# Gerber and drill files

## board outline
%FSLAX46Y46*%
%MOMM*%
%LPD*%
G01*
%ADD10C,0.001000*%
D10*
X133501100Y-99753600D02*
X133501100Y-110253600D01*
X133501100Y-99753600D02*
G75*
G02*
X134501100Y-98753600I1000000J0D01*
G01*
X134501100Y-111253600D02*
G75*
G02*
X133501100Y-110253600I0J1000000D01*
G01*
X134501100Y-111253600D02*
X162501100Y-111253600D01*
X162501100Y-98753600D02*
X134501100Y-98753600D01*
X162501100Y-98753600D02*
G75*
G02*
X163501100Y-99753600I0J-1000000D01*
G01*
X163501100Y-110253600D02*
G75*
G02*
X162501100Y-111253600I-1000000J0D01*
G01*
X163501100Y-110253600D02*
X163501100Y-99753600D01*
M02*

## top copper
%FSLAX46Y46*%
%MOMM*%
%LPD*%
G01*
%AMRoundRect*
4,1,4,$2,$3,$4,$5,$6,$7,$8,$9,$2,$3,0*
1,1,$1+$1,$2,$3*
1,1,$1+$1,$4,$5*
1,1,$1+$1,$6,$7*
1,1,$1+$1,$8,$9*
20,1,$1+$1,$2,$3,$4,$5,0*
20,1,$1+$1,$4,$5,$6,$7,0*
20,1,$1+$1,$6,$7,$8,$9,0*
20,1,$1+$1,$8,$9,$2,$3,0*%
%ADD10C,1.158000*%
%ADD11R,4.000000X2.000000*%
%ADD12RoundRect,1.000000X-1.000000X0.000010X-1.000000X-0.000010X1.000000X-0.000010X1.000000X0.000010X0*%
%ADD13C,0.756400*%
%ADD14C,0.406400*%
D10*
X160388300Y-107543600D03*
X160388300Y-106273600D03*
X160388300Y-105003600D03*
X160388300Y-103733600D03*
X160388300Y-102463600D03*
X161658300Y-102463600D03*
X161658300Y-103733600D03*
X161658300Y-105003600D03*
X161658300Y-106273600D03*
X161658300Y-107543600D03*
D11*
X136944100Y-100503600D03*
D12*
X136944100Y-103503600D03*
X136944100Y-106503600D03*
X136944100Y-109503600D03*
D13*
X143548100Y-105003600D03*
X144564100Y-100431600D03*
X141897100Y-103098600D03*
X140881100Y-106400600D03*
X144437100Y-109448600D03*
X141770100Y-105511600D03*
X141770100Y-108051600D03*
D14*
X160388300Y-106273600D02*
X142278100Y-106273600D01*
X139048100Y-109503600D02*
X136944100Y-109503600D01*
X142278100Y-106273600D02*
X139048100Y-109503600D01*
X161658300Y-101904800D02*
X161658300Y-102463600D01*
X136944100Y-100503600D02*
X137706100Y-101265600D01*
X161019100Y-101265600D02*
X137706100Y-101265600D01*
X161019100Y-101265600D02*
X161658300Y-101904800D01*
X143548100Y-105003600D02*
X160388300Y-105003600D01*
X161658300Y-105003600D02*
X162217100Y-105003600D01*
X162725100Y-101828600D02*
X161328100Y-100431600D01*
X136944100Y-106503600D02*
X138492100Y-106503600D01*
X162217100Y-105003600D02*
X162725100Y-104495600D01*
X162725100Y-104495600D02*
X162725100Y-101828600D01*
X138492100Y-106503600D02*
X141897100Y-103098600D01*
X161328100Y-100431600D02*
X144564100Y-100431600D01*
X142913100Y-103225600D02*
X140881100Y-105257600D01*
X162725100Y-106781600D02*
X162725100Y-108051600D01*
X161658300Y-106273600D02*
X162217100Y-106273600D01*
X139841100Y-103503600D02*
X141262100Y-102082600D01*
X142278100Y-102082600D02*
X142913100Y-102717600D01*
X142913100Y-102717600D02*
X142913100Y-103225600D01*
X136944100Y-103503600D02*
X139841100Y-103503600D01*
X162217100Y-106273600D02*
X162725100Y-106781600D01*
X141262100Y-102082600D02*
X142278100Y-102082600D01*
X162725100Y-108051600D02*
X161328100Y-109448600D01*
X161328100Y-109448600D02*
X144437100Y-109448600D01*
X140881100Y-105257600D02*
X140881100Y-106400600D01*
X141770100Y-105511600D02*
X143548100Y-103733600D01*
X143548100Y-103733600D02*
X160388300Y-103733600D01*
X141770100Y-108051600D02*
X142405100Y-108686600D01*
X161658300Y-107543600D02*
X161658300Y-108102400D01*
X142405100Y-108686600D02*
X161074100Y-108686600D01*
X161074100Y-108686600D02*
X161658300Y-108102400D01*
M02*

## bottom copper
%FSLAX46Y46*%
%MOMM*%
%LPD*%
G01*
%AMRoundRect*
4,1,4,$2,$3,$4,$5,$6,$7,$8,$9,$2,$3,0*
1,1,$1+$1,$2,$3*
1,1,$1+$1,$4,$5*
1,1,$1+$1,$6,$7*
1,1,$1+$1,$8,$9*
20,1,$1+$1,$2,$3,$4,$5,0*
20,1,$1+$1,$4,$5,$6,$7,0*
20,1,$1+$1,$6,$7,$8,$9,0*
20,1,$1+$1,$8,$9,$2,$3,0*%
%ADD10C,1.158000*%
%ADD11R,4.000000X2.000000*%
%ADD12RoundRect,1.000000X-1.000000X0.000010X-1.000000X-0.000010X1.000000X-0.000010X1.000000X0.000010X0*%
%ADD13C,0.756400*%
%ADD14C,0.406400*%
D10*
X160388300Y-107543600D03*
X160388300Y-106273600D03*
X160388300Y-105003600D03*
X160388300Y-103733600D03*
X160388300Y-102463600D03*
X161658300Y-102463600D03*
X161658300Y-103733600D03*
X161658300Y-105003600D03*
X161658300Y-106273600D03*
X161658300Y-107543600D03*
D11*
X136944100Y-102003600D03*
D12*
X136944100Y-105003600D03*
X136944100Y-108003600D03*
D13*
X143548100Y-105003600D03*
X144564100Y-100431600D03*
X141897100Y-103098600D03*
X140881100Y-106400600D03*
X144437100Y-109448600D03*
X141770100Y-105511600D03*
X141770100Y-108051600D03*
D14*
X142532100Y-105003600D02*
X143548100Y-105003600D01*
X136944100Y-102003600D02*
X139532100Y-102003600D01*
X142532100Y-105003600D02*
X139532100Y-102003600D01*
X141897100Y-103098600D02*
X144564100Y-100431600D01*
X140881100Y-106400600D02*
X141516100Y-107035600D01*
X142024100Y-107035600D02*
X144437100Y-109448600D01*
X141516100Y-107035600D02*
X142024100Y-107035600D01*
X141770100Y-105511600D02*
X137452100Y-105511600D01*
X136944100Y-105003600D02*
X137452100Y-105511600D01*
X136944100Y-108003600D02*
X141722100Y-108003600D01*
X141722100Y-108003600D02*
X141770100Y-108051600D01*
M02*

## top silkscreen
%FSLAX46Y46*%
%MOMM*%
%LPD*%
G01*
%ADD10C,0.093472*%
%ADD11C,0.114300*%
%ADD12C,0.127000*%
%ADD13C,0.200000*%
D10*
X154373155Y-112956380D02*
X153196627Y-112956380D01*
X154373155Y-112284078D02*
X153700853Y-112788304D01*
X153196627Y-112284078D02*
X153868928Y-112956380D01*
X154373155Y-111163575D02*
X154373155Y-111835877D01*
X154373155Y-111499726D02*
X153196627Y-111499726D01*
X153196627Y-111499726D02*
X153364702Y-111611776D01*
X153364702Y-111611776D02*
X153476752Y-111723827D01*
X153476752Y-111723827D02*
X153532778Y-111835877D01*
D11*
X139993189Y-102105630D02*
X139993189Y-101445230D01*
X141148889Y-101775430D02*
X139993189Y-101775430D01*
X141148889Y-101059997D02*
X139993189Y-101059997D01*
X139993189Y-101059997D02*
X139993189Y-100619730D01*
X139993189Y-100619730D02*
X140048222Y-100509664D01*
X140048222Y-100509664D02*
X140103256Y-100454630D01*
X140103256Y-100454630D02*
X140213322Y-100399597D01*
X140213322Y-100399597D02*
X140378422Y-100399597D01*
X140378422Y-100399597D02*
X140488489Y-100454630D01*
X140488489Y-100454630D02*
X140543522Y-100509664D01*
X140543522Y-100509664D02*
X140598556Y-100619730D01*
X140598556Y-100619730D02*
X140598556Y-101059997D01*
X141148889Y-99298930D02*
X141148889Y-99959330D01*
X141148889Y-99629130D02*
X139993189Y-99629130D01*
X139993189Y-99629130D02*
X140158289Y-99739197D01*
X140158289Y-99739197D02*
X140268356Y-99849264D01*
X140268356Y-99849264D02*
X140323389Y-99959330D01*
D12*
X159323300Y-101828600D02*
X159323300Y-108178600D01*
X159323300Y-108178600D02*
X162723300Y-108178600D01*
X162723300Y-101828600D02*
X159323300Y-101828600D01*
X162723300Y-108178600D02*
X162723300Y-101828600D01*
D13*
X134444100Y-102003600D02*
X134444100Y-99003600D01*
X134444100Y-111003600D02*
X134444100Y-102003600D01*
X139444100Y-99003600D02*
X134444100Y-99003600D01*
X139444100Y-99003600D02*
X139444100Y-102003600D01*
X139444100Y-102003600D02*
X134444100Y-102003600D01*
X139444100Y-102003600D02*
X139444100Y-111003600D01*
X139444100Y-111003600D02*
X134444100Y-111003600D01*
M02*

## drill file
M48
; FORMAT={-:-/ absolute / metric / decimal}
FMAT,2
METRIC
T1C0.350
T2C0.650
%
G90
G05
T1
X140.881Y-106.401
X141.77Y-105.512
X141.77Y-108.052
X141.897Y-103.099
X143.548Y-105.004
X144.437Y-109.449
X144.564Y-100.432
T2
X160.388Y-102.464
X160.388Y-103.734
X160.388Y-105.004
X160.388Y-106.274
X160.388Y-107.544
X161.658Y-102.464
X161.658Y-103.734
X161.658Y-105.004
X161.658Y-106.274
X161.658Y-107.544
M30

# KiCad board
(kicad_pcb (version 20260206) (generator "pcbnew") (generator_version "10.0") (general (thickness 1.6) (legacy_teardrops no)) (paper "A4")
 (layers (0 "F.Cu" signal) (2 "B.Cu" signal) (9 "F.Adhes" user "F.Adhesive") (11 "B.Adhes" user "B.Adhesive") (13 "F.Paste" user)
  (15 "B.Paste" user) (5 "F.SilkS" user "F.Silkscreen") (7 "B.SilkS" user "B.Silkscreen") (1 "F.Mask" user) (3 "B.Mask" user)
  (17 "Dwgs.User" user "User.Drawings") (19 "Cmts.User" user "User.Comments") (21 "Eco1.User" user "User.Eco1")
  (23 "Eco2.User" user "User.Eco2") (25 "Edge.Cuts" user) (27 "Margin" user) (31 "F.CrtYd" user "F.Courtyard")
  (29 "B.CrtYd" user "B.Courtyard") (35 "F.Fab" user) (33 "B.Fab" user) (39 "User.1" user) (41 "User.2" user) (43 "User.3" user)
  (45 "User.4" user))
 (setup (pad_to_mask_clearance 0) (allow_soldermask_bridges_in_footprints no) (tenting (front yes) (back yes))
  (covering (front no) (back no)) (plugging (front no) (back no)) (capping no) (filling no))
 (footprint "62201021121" (layer "F.Cu") (at 161.0233 105.0036 90)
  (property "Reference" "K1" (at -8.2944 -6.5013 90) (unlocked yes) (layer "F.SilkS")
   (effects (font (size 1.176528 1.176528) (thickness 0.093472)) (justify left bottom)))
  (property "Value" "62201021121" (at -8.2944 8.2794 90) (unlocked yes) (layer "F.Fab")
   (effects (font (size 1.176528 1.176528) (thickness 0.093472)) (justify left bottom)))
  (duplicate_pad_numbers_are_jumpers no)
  (fp_line (start 3.175 -1.7) (end -3.175 -1.7) (stroke (width 0.127) (type solid)) (layer "F.SilkS"))
  (fp_line (start -3.175 -1.7) (end -3.175 1.7) (stroke (width 0.127) (type solid)) (layer "F.SilkS"))
  (fp_line (start 3.175 1.7) (end 3.175 -1.7) (stroke (width 0.127) (type solid)) (layer "F.SilkS"))
  (fp_line (start -3.175 1.7) (end 3.175 1.7) (stroke (width 0.127) (type solid)) (layer "F.SilkS"))
  (pad "1" thru_hole circle (at -2.54 -0.635 90) (size 1.158 1.158) (drill 0.65) (layers "*.Cu" "*.Mask") (remove_unused_layers no)
   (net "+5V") (solder_mask_margin 0.1016) (thermal_bridge_angle 0))
  (pad "2" thru_hole circle (at -1.27 -0.635 90) (size 1.158 1.158) (drill 0.65) (layers "*.Cu" "*.Mask") (remove_unused_layers no)
   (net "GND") (solder_mask_margin 0.1016) (thermal_bridge_angle 0))
  (pad "3" thru_hole circle (at 0 -0.635 90) (size 1.158 1.158) (drill 0.65) (layers "*.Cu" "*.Mask") (remove_unused_layers no)
   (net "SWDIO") (solder_mask_margin 0.1016) (thermal_bridge_angle 0))
  (pad "4" thru_hole circle (at 1.27 -0.635 90) (size 1.158 1.158) (drill 0.65) (layers "*.Cu" "*.Mask") (remove_unused_layers no)
   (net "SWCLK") (solder_mask_margin 0.1016) (thermal_bridge_angle 0))
  (pad "5" thru_hole circle (at 2.54 -0.635 90) (size 1.158 1.158) (drill 0.65) (layers "*.Cu" "*.Mask") (remove_unused_layers no)
   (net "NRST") (solder_mask_margin 0.1016) (thermal_bridge_angle 0))
  (pad "6" thru_hole circle (at 2.54 0.635 90) (size 1.158 1.158) (drill 0.65) (layers "*.Cu" "*.Mask") (remove_unused_layers no)
   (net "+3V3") (solder_mask_margin 0.1016) (thermal_bridge_angle 0))
  (pad "7" thru_hole circle (at 1.27 0.635 90) (size 1.158 1.158) (drill 0.65) (layers "*.Cu" "*.Mask") (remove_unused_layers no)
   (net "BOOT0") (solder_mask_margin 0.1016) (thermal_bridge_angle 0))
  (pad "8" thru_hole circle (at 0 0.635 90) (size 1.158 1.158) (drill 0.65) (layers "*.Cu" "*.Mask") (remove_unused_layers no)
   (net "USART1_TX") (solder_mask_margin 0.1016) (thermal_bridge_angle 0))
  (pad "9" thru_hole circle (at -1.27 0.635 90) (size 1.158 1.158) (drill 0.65) (layers "*.Cu" "*.Mask") (remove_unused_layers no)
   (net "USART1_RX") (solder_mask_margin 0.1016) (thermal_bridge_angle 0))
  (pad "10" thru_hole circle (at -2.54 0.635 90) (size 1.158 1.158) (drill 0.65) (layers "*.Cu" "*.Mask") (remove_unused_layers no)
   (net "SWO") (solder_mask_margin 0.1016) (thermal_bridge_angle 0)))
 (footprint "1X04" (layer "F.Cu") (at 136.9441 105.0036 -90)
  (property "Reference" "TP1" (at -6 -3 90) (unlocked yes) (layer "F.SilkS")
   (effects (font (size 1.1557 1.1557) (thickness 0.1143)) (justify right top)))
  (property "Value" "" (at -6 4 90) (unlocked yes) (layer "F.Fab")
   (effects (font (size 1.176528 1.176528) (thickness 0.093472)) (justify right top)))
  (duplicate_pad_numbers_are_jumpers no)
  (fp_line (start -3 2.5) (end -6 2.5) (stroke (width 0.2) (type solid)) (layer "F.SilkS"))
  (fp_line (start 6 2.5) (end -3 2.5) (stroke (width 0.2) (type solid)) (layer "F.SilkS"))
  (fp_line (start -6 -2.5) (end -6 2.5) (stroke (width 0.2) (type solid)) (layer "F.SilkS"))
  (fp_line (start -6 -2.5) (end -3 -2.5) (stroke (width 0.2) (type solid)) (layer "F.SilkS"))
  (fp_line (start -3 -2.5) (end -3 2.5) (stroke (width 0.2) (type solid)) (layer "F.SilkS"))
  (fp_line (start -3 -2.5) (end 6 -2.5) (stroke (width 0.2) (type solid)) (layer "F.SilkS"))
  (fp_line (start 6 -2.5) (end 6 2.5) (stroke (width 0.2) (type solid)) (layer "F.SilkS"))
  (pad "1" smd rect (at -4.5 0 270) (size 2 4) (layers "F.Cu" "F.Mask" "F.Paste") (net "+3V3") (solder_mask_margin 0.1016)
   (solder_paste_margin 0) (thermal_bridge_angle 0))
  (pad "2" smd roundrect (at -1.5 0 270) (size 2 4) (layers "F.Cu" "F.Mask" "F.Paste") (roundrect_rratio 0.5) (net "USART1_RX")
   (solder_mask_margin 0.1016) (solder_paste_margin 0) (thermal_bridge_angle 0))
  (pad "3" smd roundrect (at 1.5 0 270) (size 2 4) (layers "F.Cu" "F.Mask" "F.Paste") (roundrect_rratio 0.5) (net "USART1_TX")
   (solder_mask_margin 0.1016) (solder_paste_margin 0) (thermal_bridge_angle 0))
  (pad "4" smd roundrect (at 4.5 0 270) (size 2 4) (layers "F.Cu" "F.Mask" "F.Paste") (roundrect_rratio 0.5) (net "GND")
   (solder_mask_margin 0.1016) (solder_paste_margin 0) (thermal_bridge_angle 0)))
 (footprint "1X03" (layer "B.Cu") (at 136.9441 105.0036 -90)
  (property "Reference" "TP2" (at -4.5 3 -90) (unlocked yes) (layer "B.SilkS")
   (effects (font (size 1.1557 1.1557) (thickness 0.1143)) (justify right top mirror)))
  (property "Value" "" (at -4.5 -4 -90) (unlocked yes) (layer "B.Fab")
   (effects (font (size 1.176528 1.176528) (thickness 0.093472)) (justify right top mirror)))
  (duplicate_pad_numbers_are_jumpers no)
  (pad "1" smd rect (at -3 0 270) (size 2 4) (layers "B.Cu" "B.Mask" "B.Paste") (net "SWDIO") (solder_mask_margin 0.1016)
   (solder_paste_margin 0) (thermal_bridge_angle 0))
  (pad "2" smd roundrect (at 0 0 270) (size 2 4) (layers "B.Cu" "B.Mask" "B.Paste") (roundrect_rratio 0.5) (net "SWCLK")
   (solder_mask_margin 0.1016) (solder_paste_margin 0) (thermal_bridge_angle 0))
  (pad "3" smd roundrect (at 3 0 270) (size 2 4) (layers "B.Cu" "B.Mask" "B.Paste") (roundrect_rratio 0.5) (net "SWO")
   (solder_mask_margin 0.1016) (solder_paste_margin 0) (thermal_bridge_angle 0)))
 (gr_line (start 133.5011 99.7536) (end 133.5011 110.2536) (stroke (width 0.001) (type solid)) (layer "Edge.Cuts"))
 (gr_arc (start 133.5011 99.7536) (mid 133.793993 99.046493) (end 134.5011 98.7536) (stroke (width 0.001) (type solid)) (layer "Edge.Cuts"))
 (gr_arc (start 134.5011 111.2536) (mid 133.793993 110.960707) (end 133.5011 110.2536) (stroke (width 0.001) (type solid))
  (layer "Edge.Cuts"))
 (gr_line (start 134.5011 111.2536) (end 162.5011 111.2536) (stroke (width 0.001) (type solid)) (layer "Edge.Cuts"))
 (gr_line (start 162.5011 98.7536) (end 134.5011 98.7536) (stroke (width 0.001) (type solid)) (layer "Edge.Cuts"))
 (gr_arc (start 162.5011 98.7536) (mid 163.208207 99.046493) (end 163.5011 99.7536) (stroke (width 0.001) (type solid)) (layer "Edge.Cuts"))
 (gr_arc (start 163.5011 110.2536) (mid 163.208207 110.960707) (end 162.5011 111.2536) (stroke (width 0.001) (type solid))
  (layer "Edge.Cuts"))
 (gr_line (start 163.5011 110.2536) (end 163.5011 99.7536) (stroke (width 0.001) (type solid)) (layer "Edge.Cuts"))
 (segment (start 160.3883 106.2736) (end 142.2781 106.2736) (width 0.4064) (layer "F.Cu") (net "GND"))
 (segment (start 139.0481 109.5036) (end 136.9441 109.5036) (width 0.4064) (layer "F.Cu") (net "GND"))
 (segment (start 142.2781 106.2736) (end 139.0481 109.5036) (width 0.4064) (layer "F.Cu") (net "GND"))
 (segment (start 161.6583 101.9048) (end 161.6583 102.4636) (width 0.4064) (layer "F.Cu") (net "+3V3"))
 (segment (start 136.9441 100.5036) (end 137.7061 101.2656) (width 0.4064) (layer "F.Cu") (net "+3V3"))
 (segment (start 161.0191 101.2656) (end 137.7061 101.2656) (width 0.4064) (layer "F.Cu") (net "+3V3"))
 (segment (start 161.0191 101.2656) (end 161.6583 101.9048) (width 0.4064) (layer "F.Cu") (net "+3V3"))
 (segment (start 143.5481 105.0036) (end 160.3883 105.0036) (width 0.4064) (layer "F.Cu") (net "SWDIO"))
 (via (at 143.5481 105.0036) (size 0.7564) (drill 0.35) (layers "F.Cu" "B.Cu") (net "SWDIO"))
 (segment (start 142.5321 105.0036) (end 143.5481 105.0036) (width 0.4064) (layer "B.Cu") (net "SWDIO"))
 (segment (start 136.9441 102.0036) (end 139.5321 102.0036) (width 0.4064) (layer "B.Cu") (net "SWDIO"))
 (segment (start 142.5321 105.0036) (end 139.5321 102.0036) (width 0.4064) (layer "B.Cu") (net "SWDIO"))
 (segment (start 161.6583 105.0036) (end 162.2171 105.0036) (width 0.4064) (layer "F.Cu") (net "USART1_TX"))
 (segment (start 162.7251 101.8286) (end 161.3281 100.4316) (width 0.4064) (layer "F.Cu") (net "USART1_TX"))
 (segment (start 136.9441 106.5036) (end 138.4921 106.5036) (width 0.4064) (layer "F.Cu") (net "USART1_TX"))
 (segment (start 162.2171 105.0036) (end 162.7251 104.4956) (width 0.4064) (layer "F.Cu") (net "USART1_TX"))
 (segment (start 162.7251 104.4956) (end 162.7251 101.8286) (width 0.4064) (layer "F.Cu") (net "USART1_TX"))
 (segment (start 138.4921 106.5036) (end 141.8971 103.0986) (width 0.4064) (layer "F.Cu") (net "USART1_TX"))
 (segment (start 161.3281 100.4316) (end 144.5641 100.4316) (width 0.4064) (layer "F.Cu") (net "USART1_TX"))
 (via (at 144.5641 100.4316) (size 0.7564) (drill 0.35) (layers "F.Cu" "B.Cu") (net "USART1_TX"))
 (via (at 141.8971 103.0986) (size 0.7564) (drill 0.35) (layers "F.Cu" "B.Cu") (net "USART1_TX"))
 (segment (start 141.8971 103.0986) (end 144.5641 100.4316) (width 0.4064) (layer "B.Cu") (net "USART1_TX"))
 (segment (start 142.9131 103.2256) (end 140.8811 105.2576) (width 0.4064) (layer "F.Cu") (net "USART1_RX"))
 (segment (start 162.7251 106.7816) (end 162.7251 108.0516) (width 0.4064) (layer "F.Cu") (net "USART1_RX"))
 (segment (start 161.6583 106.2736) (end 162.2171 106.2736) (width 0.4064) (layer "F.Cu") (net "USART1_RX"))
 (segment (start 139.8411 103.5036) (end 141.2621 102.0826) (width 0.4064) (layer "F.Cu") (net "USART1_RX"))
 (segment (start 142.2781 102.0826) (end 142.9131 102.7176) (width 0.4064) (layer "F.Cu") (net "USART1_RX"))
 (segment (start 142.9131 102.7176) (end 142.9131 103.2256) (width 0.4064) (layer "F.Cu") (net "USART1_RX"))
 (segment (start 136.9441 103.5036) (end 139.8411 103.5036) (width 0.4064) (layer "F.Cu") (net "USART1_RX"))
 (segment (start 162.2171 106.2736) (end 162.7251 106.7816) (width 0.4064) (layer "F.Cu") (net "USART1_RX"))
 (segment (start 141.2621 102.0826) (end 142.2781 102.0826) (width 0.4064) (layer "F.Cu") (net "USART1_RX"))
 (segment (start 162.7251 108.0516) (end 161.3281 109.4486) (width 0.4064) (layer "F.Cu") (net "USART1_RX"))
 (segment (start 161.3281 109.4486) (end 144.4371 109.4486) (width 0.4064) (layer "F.Cu") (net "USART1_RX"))
 (segment (start 140.8811 105.2576) (end 140.8811 106.4006) (width 0.4064) (layer "F.Cu") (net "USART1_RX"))
 (via (at 140.8811 106.4006) (size 0.7564) (drill 0.35) (layers "F.Cu" "B.Cu") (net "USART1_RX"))
 (via (at 144.4371 109.4486) (size 0.7564) (drill 0.35) (layers "F.Cu" "B.Cu") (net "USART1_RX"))
 (segment (start 140.8811 106.4006) (end 141.5161 107.0356) (width 0.4064) (layer "B.Cu") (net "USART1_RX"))
 (segment (start 142.0241 107.0356) (end 144.4371 109.4486) (width 0.4064) (layer "B.Cu") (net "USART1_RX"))
 (segment (start 141.5161 107.0356) (end 142.0241 107.0356) (width 0.4064) (layer "B.Cu") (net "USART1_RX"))
 (segment (start 141.7701 105.5116) (end 143.5481 103.7336) (width 0.4064) (layer "F.Cu") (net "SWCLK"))
 (segment (start 143.5481 103.7336) (end 160.3883 103.7336) (width 0.4064) (layer "F.Cu") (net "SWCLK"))
 (via (at 141.7701 105.5116) (size 0.7564) (drill 0.35) (layers "F.Cu" "B.Cu") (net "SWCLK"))
 (segment (start 141.7701 105.5116) (end 137.4521 105.5116) (width 0.4064) (layer "B.Cu") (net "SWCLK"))
 (segment (start 136.9441 105.0036) (end 137.4521 105.5116) (width 0.4064) (layer "B.Cu") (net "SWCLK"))
 (segment (start 141.7701 108.0516) (end 142.4051 108.6866) (width 0.4064) (layer "F.Cu") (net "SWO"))
 (segment (start 161.6583 107.5436) (end 161.6583 108.1024) (width 0.4064) (layer "F.Cu") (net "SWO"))
 (segment (start 142.4051 108.6866) (end 161.0741 108.6866) (width 0.4064) (layer "F.Cu") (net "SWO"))
 (segment (start 161.0741 108.6866) (end 161.6583 108.1024) (width 0.4064) (layer "F.Cu") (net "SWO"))
 (via (at 141.7701 108.0516) (size 0.7564) (drill 0.35) (layers "F.Cu" "B.Cu") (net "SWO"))
 (segment (start 136.9441 108.0036) (end 141.7221 108.0036) (width 0.4064) (layer "B.Cu") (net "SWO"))
 (segment (start 141.7221 108.0036) (end 141.7701 108.0516) (width 0.4064) (layer "B.Cu") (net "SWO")))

